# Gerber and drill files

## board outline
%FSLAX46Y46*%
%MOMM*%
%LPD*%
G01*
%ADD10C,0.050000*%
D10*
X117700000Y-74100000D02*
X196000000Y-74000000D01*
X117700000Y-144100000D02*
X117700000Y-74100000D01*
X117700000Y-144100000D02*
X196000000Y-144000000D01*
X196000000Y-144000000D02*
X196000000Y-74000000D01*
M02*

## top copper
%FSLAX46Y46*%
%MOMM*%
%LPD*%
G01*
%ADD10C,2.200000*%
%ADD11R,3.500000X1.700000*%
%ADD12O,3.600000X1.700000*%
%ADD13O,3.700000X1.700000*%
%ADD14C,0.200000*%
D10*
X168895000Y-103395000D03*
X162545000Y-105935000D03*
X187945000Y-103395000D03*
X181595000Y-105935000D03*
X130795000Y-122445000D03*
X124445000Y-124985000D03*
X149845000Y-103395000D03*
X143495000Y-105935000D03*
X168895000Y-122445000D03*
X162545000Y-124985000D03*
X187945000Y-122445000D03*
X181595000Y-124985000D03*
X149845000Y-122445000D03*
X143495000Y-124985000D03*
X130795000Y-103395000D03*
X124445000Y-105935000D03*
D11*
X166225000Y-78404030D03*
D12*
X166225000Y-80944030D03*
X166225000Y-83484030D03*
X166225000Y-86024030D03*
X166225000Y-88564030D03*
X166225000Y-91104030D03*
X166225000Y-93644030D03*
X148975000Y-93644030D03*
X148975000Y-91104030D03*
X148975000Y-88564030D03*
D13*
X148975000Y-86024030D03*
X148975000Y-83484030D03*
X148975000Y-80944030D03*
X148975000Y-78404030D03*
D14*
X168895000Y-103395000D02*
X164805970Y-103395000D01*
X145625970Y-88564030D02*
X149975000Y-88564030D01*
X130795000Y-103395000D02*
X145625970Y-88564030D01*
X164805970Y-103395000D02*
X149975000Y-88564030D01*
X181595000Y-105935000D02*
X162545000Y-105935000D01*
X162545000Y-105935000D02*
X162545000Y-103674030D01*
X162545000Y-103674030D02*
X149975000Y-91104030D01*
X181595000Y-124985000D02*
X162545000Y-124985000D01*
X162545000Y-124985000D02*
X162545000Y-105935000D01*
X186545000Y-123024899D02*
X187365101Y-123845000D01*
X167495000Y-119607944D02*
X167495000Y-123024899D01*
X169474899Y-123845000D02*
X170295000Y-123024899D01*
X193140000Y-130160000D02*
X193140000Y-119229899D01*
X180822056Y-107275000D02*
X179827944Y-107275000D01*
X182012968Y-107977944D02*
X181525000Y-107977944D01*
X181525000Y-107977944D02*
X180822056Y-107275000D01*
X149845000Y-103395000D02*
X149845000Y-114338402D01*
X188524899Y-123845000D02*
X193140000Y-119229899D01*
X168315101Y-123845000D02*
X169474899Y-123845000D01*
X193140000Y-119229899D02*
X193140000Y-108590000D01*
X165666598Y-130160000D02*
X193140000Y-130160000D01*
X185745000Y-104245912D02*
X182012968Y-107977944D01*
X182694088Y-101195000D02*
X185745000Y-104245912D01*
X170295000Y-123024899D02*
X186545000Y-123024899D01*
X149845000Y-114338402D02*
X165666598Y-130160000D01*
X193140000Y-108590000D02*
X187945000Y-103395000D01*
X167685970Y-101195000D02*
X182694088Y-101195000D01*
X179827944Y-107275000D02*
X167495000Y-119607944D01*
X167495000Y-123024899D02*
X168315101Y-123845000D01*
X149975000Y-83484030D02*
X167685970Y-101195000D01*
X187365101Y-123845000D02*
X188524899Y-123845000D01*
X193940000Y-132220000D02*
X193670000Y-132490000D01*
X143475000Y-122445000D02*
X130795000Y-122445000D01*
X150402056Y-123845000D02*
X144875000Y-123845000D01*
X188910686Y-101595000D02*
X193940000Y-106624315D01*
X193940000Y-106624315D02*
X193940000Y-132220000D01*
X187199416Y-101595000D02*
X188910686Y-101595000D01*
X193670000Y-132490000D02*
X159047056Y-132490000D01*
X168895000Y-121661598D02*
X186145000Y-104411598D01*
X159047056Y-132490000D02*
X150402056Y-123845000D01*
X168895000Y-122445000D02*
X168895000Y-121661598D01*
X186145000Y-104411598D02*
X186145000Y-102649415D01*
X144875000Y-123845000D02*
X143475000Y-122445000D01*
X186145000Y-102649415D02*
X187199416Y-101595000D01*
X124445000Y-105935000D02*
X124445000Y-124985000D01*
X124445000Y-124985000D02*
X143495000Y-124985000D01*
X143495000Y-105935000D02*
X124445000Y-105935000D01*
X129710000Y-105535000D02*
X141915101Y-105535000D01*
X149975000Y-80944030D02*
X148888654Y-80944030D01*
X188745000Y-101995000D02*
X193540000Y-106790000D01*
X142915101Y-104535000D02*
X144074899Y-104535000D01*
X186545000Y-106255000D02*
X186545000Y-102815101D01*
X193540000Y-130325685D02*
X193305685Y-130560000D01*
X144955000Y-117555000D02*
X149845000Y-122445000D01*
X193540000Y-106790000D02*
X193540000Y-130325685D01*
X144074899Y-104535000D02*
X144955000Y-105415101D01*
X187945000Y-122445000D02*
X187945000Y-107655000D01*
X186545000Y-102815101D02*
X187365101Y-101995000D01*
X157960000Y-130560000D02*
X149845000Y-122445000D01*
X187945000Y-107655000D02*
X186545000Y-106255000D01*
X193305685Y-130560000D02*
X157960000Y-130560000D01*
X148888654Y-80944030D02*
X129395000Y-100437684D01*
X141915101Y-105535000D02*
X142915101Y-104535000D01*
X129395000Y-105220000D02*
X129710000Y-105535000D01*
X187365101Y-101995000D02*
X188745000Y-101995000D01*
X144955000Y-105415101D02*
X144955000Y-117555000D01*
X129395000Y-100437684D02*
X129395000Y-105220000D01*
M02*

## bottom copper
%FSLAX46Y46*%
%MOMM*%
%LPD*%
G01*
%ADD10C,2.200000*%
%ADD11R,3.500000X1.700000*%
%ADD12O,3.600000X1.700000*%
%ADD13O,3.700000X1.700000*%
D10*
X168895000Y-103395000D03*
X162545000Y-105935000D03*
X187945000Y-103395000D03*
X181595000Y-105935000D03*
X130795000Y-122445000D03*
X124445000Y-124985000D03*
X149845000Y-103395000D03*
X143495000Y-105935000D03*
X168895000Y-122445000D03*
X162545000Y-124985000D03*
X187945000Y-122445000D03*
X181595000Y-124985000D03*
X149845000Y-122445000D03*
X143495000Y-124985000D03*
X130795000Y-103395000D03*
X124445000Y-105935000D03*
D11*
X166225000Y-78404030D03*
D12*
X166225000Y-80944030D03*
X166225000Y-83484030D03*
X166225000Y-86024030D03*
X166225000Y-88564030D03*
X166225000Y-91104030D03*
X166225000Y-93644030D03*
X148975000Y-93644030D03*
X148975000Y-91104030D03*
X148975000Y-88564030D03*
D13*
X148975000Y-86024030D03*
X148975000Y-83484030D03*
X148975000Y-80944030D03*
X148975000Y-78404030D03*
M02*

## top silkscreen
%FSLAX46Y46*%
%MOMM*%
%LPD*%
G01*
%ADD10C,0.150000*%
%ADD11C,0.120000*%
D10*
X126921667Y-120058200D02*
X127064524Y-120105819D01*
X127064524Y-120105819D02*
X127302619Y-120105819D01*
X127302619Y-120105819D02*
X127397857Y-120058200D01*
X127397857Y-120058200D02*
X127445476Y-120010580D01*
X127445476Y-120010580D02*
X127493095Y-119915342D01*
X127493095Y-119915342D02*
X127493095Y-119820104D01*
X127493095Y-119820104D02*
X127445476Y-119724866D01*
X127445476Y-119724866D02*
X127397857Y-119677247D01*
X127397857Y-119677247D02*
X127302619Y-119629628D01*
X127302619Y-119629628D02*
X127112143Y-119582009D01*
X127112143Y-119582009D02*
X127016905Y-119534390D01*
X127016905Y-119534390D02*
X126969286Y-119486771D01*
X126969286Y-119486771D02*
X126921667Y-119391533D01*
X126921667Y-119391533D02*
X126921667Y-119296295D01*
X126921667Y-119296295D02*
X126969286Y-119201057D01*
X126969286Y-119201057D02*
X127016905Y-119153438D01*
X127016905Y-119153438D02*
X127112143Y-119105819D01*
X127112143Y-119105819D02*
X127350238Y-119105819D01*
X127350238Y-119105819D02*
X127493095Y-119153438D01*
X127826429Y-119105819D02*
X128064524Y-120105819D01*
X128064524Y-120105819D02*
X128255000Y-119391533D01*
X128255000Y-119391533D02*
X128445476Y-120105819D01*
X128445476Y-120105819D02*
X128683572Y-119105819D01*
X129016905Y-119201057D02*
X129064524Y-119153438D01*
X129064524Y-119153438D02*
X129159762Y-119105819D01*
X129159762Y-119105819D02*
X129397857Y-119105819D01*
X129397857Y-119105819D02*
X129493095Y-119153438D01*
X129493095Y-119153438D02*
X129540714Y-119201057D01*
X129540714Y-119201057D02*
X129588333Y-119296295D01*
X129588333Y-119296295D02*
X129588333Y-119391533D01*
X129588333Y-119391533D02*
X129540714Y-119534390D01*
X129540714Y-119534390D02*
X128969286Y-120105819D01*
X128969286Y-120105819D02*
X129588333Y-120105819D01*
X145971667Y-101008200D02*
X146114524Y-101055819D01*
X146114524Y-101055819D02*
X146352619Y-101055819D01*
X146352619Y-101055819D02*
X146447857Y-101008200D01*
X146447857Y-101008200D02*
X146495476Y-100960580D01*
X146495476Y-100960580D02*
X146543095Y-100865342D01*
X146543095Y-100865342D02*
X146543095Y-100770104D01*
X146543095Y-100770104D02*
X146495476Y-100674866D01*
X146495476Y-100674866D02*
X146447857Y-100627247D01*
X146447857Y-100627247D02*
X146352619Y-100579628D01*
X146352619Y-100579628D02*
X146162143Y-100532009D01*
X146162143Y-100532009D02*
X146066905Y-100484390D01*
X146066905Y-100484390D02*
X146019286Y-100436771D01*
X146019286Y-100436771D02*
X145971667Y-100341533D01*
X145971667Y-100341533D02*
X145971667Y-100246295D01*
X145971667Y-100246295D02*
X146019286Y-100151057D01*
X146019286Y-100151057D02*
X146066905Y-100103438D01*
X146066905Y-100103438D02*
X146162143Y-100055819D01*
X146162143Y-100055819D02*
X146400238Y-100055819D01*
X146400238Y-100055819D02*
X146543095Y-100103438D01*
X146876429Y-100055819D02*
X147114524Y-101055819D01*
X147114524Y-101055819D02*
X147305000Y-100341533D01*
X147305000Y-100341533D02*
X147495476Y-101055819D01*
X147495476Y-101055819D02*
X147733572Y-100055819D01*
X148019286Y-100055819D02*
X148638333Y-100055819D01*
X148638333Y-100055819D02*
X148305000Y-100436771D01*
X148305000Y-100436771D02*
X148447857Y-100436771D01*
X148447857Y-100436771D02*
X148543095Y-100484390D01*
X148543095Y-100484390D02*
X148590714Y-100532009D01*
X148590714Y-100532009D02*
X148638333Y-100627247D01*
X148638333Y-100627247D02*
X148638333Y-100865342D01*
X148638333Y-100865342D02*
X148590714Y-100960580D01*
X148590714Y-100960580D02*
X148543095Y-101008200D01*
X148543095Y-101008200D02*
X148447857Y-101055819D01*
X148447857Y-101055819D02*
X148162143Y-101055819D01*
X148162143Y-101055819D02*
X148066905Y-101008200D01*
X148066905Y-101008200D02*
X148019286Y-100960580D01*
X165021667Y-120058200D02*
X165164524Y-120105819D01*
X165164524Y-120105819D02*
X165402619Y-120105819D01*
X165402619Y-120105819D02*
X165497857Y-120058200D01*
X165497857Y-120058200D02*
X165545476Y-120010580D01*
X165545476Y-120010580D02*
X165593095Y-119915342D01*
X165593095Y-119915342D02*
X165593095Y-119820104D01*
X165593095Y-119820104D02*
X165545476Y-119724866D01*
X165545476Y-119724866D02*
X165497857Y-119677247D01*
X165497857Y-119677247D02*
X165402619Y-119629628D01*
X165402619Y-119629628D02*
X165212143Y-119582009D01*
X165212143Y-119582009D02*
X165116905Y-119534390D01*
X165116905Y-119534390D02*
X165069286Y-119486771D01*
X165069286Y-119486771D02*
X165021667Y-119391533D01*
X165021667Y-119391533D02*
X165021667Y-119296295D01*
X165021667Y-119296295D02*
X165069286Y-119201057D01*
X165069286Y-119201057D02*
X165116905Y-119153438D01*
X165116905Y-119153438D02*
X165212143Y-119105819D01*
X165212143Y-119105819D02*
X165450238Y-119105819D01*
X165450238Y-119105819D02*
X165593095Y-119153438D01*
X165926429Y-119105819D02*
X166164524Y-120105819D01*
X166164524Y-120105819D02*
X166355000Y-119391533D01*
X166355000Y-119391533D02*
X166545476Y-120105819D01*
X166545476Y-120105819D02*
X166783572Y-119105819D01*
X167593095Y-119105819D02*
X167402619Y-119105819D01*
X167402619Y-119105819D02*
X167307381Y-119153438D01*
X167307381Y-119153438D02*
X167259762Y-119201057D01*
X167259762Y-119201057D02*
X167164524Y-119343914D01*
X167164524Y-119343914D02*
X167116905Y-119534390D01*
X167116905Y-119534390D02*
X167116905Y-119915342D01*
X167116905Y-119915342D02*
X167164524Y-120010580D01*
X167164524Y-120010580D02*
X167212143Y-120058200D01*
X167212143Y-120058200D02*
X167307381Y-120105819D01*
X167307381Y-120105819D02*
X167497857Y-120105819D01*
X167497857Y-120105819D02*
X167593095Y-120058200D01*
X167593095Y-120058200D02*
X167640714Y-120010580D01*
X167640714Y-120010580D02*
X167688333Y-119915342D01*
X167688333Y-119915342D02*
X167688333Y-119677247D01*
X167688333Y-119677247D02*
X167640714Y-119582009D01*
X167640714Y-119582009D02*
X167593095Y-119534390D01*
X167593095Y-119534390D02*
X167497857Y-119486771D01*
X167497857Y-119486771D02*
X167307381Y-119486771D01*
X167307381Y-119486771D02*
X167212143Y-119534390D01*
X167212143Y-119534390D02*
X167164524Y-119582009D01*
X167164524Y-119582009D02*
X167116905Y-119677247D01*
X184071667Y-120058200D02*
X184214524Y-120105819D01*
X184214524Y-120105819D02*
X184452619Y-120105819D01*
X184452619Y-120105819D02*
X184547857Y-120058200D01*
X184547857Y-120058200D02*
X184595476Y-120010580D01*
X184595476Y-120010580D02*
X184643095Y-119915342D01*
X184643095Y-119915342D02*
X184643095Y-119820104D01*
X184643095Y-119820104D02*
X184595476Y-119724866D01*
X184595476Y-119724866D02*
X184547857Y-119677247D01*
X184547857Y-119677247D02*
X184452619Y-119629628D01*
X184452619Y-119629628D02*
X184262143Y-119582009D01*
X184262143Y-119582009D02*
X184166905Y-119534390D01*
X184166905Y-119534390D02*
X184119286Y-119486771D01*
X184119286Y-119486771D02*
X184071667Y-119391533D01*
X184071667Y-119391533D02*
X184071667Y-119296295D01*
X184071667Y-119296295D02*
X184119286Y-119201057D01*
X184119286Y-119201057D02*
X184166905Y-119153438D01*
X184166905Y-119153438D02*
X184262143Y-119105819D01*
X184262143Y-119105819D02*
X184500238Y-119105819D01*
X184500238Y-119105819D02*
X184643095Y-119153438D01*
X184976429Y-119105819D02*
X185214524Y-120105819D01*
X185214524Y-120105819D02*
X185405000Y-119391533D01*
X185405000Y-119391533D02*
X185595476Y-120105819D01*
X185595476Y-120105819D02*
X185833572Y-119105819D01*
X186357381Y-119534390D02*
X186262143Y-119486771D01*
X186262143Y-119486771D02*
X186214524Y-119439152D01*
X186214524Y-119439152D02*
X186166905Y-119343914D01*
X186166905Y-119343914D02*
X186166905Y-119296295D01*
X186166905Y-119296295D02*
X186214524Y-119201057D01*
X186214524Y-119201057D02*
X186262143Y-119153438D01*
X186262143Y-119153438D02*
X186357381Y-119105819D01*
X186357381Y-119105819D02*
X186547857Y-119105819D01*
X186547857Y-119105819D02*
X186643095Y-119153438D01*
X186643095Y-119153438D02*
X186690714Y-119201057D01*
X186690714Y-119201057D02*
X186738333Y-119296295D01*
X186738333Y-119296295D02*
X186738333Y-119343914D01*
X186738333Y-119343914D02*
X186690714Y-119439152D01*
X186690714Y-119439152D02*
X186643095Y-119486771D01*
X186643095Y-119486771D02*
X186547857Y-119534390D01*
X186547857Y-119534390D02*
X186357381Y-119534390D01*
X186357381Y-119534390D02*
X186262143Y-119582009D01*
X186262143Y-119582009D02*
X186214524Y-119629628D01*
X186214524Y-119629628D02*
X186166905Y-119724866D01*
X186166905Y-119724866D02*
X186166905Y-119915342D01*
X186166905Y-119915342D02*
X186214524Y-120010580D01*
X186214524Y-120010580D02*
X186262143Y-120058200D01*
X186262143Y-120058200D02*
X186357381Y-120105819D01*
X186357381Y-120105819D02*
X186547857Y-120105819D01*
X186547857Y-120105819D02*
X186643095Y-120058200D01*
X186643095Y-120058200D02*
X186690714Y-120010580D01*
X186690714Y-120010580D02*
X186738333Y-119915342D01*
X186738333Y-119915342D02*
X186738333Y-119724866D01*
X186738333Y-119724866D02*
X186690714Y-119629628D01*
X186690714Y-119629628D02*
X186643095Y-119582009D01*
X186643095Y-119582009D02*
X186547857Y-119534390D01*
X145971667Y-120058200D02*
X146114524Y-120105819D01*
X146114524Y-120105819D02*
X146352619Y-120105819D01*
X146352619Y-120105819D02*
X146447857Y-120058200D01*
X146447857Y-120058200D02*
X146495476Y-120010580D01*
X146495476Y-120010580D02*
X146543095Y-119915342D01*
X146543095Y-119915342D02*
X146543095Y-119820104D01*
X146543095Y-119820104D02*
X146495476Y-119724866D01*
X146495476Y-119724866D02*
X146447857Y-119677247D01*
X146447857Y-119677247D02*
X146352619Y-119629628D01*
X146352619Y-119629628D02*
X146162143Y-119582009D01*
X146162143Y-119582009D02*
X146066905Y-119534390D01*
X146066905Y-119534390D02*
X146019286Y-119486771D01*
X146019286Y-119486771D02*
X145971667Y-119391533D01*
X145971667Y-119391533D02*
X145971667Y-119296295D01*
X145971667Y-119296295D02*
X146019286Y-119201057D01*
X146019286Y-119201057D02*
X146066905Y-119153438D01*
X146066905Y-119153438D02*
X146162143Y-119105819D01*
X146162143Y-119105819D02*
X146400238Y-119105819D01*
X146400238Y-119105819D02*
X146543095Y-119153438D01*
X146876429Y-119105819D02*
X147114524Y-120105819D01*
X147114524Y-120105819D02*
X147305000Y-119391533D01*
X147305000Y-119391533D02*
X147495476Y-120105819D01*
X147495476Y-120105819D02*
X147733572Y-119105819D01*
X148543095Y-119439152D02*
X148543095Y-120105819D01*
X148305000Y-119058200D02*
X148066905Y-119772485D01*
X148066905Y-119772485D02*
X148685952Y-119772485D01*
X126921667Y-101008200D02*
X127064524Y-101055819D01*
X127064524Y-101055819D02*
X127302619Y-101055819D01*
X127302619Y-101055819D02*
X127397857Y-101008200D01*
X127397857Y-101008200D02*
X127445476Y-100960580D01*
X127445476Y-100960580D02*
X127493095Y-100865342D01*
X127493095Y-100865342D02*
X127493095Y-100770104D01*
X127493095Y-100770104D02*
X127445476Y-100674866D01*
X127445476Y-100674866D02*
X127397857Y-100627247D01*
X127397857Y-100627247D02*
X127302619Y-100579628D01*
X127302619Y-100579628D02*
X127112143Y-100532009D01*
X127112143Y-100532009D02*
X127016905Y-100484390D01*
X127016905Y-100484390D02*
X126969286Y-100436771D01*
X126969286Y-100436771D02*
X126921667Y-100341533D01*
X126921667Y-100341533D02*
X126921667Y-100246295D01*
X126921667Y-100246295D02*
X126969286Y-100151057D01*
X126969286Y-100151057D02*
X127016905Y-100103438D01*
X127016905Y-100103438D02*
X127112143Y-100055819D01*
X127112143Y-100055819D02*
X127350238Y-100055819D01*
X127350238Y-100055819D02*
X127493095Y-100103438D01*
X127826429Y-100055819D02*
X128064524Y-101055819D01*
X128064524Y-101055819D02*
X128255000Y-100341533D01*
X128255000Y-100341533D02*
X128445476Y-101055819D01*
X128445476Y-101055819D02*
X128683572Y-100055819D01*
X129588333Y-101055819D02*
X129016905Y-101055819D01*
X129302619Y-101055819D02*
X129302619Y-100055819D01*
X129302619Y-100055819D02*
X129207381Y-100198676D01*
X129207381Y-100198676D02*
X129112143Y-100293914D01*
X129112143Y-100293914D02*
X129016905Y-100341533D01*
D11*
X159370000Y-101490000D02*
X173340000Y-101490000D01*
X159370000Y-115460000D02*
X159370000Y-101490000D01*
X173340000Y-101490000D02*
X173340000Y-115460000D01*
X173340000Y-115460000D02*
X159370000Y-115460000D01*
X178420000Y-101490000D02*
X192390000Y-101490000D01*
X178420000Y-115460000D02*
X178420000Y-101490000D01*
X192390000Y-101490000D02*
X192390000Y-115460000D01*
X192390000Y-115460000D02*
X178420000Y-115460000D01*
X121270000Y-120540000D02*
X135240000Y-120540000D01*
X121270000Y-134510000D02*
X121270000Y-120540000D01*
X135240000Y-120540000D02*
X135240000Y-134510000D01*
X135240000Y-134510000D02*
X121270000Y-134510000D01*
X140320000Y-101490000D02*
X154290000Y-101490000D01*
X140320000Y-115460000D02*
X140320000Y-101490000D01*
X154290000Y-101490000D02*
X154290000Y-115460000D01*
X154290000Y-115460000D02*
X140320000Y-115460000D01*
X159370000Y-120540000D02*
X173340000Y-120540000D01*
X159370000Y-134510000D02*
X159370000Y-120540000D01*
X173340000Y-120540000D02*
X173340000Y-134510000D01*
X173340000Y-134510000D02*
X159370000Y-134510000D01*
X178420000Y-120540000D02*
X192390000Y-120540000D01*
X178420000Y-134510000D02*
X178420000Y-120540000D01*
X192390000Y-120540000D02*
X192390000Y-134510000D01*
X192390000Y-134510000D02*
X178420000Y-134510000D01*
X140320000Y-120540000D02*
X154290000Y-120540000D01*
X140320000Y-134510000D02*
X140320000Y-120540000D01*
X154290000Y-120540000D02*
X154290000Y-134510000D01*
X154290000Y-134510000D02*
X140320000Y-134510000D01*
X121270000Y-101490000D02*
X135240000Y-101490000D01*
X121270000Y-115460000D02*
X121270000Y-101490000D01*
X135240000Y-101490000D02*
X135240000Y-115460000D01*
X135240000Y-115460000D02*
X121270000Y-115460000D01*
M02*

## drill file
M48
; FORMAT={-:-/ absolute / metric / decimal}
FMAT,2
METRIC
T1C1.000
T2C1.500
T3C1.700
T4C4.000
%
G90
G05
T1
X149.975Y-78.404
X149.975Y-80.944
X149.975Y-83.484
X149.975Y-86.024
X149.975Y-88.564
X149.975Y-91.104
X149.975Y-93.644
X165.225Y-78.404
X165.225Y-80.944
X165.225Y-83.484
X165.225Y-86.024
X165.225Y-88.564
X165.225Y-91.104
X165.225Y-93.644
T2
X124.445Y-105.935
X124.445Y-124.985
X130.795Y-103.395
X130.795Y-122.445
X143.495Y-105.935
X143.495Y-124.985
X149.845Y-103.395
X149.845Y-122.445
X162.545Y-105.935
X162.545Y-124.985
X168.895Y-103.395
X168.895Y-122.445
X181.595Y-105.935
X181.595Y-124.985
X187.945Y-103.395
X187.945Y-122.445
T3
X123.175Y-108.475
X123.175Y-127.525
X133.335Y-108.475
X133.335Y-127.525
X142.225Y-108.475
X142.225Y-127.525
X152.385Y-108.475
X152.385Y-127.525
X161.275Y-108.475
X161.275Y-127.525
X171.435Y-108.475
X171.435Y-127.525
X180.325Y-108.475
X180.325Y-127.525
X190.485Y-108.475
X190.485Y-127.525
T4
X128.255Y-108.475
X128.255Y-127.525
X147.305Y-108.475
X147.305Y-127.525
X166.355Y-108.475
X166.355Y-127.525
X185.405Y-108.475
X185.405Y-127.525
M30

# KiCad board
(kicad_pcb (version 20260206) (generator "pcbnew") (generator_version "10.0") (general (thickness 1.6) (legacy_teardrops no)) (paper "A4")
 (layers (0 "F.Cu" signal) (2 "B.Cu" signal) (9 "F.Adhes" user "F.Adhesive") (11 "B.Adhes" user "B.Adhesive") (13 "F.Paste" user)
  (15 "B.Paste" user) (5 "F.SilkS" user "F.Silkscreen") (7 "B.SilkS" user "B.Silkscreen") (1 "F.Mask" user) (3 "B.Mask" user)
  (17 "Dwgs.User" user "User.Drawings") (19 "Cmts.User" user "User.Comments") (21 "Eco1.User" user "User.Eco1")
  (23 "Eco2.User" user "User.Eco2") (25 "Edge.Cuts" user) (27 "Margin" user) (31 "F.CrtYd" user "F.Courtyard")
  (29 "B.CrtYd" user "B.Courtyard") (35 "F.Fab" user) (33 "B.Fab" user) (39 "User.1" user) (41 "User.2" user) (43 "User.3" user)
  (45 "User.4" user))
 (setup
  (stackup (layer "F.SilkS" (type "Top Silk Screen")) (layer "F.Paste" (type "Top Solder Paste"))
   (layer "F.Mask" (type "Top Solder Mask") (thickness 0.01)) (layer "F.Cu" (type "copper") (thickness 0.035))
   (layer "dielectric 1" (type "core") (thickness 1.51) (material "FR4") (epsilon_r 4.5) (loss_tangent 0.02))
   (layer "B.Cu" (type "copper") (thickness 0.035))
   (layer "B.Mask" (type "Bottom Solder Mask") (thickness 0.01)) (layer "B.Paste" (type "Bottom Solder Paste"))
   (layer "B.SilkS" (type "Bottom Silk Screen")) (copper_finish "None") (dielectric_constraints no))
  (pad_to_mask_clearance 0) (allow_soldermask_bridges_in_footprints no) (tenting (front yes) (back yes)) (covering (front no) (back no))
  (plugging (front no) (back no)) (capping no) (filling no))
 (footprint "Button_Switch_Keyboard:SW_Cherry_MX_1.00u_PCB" (layer "F.Cu") (at 168.895 103.395)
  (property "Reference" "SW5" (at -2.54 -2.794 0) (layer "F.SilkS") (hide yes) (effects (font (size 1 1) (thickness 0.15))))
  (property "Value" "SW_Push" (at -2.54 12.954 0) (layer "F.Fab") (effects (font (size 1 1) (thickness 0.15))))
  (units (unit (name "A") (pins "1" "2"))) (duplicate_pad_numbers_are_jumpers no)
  (fp_line (start -9.525 -1.905) (end 4.445 -1.905) (stroke (width 0.12) (type solid)) (layer "F.SilkS"))
  (fp_line (start -9.525 12.065) (end -9.525 -1.905) (stroke (width 0.12) (type solid)) (layer "F.SilkS"))
  (fp_line (start 4.445 -1.905) (end 4.445 12.065) (stroke (width 0.12) (type solid)) (layer "F.SilkS"))
  (fp_line (start 4.445 12.065) (end -9.525 12.065) (stroke (width 0.12) (type solid)) (layer "F.SilkS"))
  (pad "" np_thru_hole circle (at -7.62 5.08) (size 1.7 1.7) (drill 1.7) (layers "*.Cu" "*.Mask"))
  (pad "" np_thru_hole circle (at -2.54 5.08) (size 4 4) (drill 4) (layers "*.Cu" "*.Mask"))
  (pad "" np_thru_hole circle (at 2.54 5.08) (size 1.7 1.7) (drill 1.7) (layers "*.Cu" "*.Mask"))
  (pad "1" thru_hole circle (at 0 0) (size 2.2 2.2) (drill 1.5) (layers "*.Cu" "*.Mask") (remove_unused_layers no)
   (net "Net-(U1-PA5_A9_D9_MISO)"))
  (pad "2" thru_hole circle (at -6.35 2.54) (size 2.2 2.2) (drill 1.5) (layers "*.Cu" "*.Mask") (remove_unused_layers no)
   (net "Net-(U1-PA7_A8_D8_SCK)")))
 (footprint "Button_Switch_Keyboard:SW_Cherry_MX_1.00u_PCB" (layer "F.Cu") (at 187.945 103.395)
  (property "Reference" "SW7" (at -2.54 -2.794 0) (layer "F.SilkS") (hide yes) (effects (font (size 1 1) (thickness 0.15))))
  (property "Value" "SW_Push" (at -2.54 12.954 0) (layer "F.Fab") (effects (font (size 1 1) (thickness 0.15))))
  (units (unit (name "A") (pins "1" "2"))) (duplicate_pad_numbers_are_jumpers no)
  (fp_line (start -9.525 -1.905) (end 4.445 -1.905) (stroke (width 0.12) (type solid)) (layer "F.SilkS"))
  (fp_line (start -9.525 12.065) (end -9.525 -1.905) (stroke (width 0.12) (type solid)) (layer "F.SilkS"))
  (fp_line (start 4.445 -1.905) (end 4.445 12.065) (stroke (width 0.12) (type solid)) (layer "F.SilkS"))
  (fp_line (start 4.445 12.065) (end -9.525 12.065) (stroke (width 0.12) (type solid)) (layer "F.SilkS"))
  (pad "" np_thru_hole circle (at -7.62 5.08) (size 1.7 1.7) (drill 1.7) (layers "*.Cu" "*.Mask"))
  (pad "" np_thru_hole circle (at -2.54 5.08) (size 4 4) (drill 4) (layers "*.Cu" "*.Mask"))
  (pad "" np_thru_hole circle (at 2.54 5.08) (size 1.7 1.7) (drill 1.7) (layers "*.Cu" "*.Mask"))
  (pad "1" thru_hole circle (at 0 0) (size 2.2 2.2) (drill 1.5) (layers "*.Cu" "*.Mask") (remove_unused_layers no) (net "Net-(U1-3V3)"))
  (pad "2" thru_hole circle (at -6.35 2.54) (size 2.2 2.2) (drill 1.5) (layers "*.Cu" "*.Mask") (remove_unused_layers no)
   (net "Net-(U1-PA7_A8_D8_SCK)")))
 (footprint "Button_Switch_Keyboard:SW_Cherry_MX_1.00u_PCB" (layer "F.Cu") (at 130.795 122.445)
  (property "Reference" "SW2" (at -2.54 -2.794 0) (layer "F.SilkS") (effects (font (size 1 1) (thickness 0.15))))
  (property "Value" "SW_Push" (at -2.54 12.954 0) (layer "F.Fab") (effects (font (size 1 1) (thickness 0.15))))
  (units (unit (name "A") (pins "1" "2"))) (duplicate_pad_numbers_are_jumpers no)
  (fp_line (start -9.525 -1.905) (end 4.445 -1.905) (stroke (width 0.12) (type solid)) (layer "F.SilkS"))
  (fp_line (start -9.525 12.065) (end -9.525 -1.905) (stroke (width 0.12) (type solid)) (layer "F.SilkS"))
  (fp_line (start 4.445 -1.905) (end 4.445 12.065) (stroke (width 0.12) (type solid)) (layer "F.SilkS"))
  (fp_line (start 4.445 12.065) (end -9.525 12.065) (stroke (width 0.12) (type solid)) (layer "F.SilkS"))
  (pad "" np_thru_hole circle (at -7.62 5.08) (size 1.7 1.7) (drill 1.7) (layers "*.Cu" "*.Mask"))
  (pad "" np_thru_hole circle (at -2.54 5.08) (size 4 4) (drill 4) (layers "*.Cu" "*.Mask"))
  (pad "" np_thru_hole circle (at 2.54 5.08) (size 1.7 1.7) (drill 1.7) (layers "*.Cu" "*.Mask"))
  (pad "1" thru_hole circle (at 0 0) (size 2.2 2.2) (drill 1.5) (layers "*.Cu" "*.Mask") (remove_unused_layers no)
   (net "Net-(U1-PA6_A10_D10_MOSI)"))
  (pad "2" thru_hole circle (at -6.35 2.54) (size 2.2 2.2) (drill 1.5) (layers "*.Cu" "*.Mask") (remove_unused_layers no)
   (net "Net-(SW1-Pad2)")))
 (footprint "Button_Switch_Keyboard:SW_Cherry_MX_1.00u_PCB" (layer "F.Cu") (at 149.845 103.395)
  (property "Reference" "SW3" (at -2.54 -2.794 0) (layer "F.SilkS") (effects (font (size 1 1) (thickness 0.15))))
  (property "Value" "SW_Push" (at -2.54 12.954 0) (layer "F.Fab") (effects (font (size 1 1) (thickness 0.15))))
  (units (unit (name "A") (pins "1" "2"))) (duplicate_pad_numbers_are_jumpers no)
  (fp_line (start -9.525 -1.905) (end 4.445 -1.905) (stroke (width 0.12) (type solid)) (layer "F.SilkS"))
  (fp_line (start -9.525 12.065) (end -9.525 -1.905) (stroke (width 0.12) (type solid)) (layer "F.SilkS"))
  (fp_line (start 4.445 -1.905) (end 4.445 12.065) (stroke (width 0.12) (type solid)) (layer "F.SilkS"))
  (fp_line (start 4.445 12.065) (end -9.525 12.065) (stroke (width 0.12) (type solid)) (layer "F.SilkS"))
  (pad "" np_thru_hole circle (at -7.62 5.08) (size 1.7 1.7) (drill 1.7) (layers "*.Cu" "*.Mask"))
  (pad "" np_thru_hole circle (at -2.54 5.08) (size 4 4) (drill 4) (layers "*.Cu" "*.Mask"))
  (pad "" np_thru_hole circle (at 2.54 5.08) (size 1.7 1.7) (drill 1.7) (layers "*.Cu" "*.Mask"))
  (pad "1" thru_hole circle (at 0 0) (size 2.2 2.2) (drill 1.5) (layers "*.Cu" "*.Mask") (remove_unused_layers no) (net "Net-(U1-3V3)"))
  (pad "2" thru_hole circle (at -6.35 2.54) (size 2.2 2.2) (drill 1.5) (layers "*.Cu" "*.Mask") (remove_unused_layers no)
   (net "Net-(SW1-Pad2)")))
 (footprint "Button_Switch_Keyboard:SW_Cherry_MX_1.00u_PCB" (layer "F.Cu") (at 168.895 122.445)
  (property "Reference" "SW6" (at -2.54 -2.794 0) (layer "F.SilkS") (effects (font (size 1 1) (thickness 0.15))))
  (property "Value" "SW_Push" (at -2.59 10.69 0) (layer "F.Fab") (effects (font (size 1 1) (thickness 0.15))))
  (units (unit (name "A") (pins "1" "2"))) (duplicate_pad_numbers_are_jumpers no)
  (fp_line (start -9.525 -1.905) (end 4.445 -1.905) (stroke (width 0.12) (type solid)) (layer "F.SilkS"))
  (fp_line (start -9.525 12.065) (end -9.525 -1.905) (stroke (width 0.12) (type solid)) (layer "F.SilkS"))
  (fp_line (start 4.445 -1.905) (end 4.445 12.065) (stroke (width 0.12) (type solid)) (layer "F.SilkS"))
  (fp_line (start 4.445 12.065) (end -9.525 12.065) (stroke (width 0.12) (type solid)) (layer "F.SilkS"))
  (pad "" np_thru_hole circle (at -7.62 5.08) (size 1.7 1.7) (drill 1.7) (layers "*.Cu" "*.Mask"))
  (pad "" np_thru_hole circle (at -2.54 5.08) (size 4 4) (drill 4) (layers "*.Cu" "*.Mask"))
  (pad "" np_thru_hole circle (at 2.54 5.08) (size 1.7 1.7) (drill 1.7) (layers "*.Cu" "*.Mask"))
  (pad "1" thru_hole circle (at 0 0) (size 2.2 2.2) (drill 1.5) (layers "*.Cu" "*.Mask") (remove_unused_layers no)
   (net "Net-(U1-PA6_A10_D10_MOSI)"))
  (pad "2" thru_hole circle (at -6.35 2.54) (size 2.2 2.2) (drill 1.5) (layers "*.Cu" "*.Mask") (remove_unused_layers no)
   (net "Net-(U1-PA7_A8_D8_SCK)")))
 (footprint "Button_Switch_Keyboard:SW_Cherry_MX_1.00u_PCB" (layer "F.Cu") (at 187.945 122.445)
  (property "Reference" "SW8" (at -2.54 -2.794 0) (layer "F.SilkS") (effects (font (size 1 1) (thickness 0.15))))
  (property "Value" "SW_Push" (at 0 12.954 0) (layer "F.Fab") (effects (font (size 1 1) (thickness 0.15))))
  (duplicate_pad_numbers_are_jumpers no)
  (fp_line (start -9.525 -1.905) (end 4.445 -1.905) (stroke (width 0.12) (type solid)) (layer "F.SilkS"))
  (fp_line (start -9.525 12.065) (end -9.525 -1.905) (stroke (width 0.12) (type solid)) (layer "F.SilkS"))
  (fp_line (start 4.445 -1.905) (end 4.445 12.065) (stroke (width 0.12) (type solid)) (layer "F.SilkS"))
  (fp_line (start 4.445 12.065) (end -9.525 12.065) (stroke (width 0.12) (type solid)) (layer "F.SilkS"))
  (pad "" np_thru_hole circle (at -7.62 5.08) (size 1.7 1.7) (drill 1.7) (layers "*.Cu" "*.Mask"))
  (pad "" np_thru_hole circle (at -2.54 5.08) (size 4 4) (drill 4) (layers "*.Cu" "*.Mask"))
  (pad "" np_thru_hole circle (at 2.54 5.08) (size 1.7 1.7) (drill 1.7) (layers "*.Cu" "*.Mask"))
  (pad "1" thru_hole circle (at 0 0) (size 2.2 2.2) (drill 1.5) (layers "*.Cu" "*.Mask") (remove_unused_layers no) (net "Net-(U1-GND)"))
  (pad "2" thru_hole circle (at -6.35 2.54) (size 2.2 2.2) (drill 1.5) (layers "*.Cu" "*.Mask") (remove_unused_layers no)
   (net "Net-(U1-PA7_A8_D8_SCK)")))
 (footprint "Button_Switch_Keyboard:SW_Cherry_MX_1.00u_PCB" (layer "F.Cu") (at 149.845 122.445)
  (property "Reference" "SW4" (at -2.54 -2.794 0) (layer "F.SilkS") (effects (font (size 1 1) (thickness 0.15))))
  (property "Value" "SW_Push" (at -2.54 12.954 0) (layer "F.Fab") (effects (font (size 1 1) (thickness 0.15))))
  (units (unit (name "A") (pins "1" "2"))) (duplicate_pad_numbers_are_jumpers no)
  (fp_line (start -9.525 -1.905) (end 4.445 -1.905) (stroke (width 0.12) (type solid)) (layer "F.SilkS"))
  (fp_line (start -9.525 12.065) (end -9.525 -1.905) (stroke (width 0.12) (type solid)) (layer "F.SilkS"))
  (fp_line (start 4.445 -1.905) (end 4.445 12.065) (stroke (width 0.12) (type solid)) (layer "F.SilkS"))
  (fp_line (start 4.445 12.065) (end -9.525 12.065) (stroke (width 0.12) (type solid)) (layer "F.SilkS"))
  (pad "" np_thru_hole circle (at -7.62 5.08) (size 1.7 1.7) (drill 1.7) (layers "*.Cu" "*.Mask"))
  (pad "" np_thru_hole circle (at -2.54 5.08) (size 4 4) (drill 4) (layers "*.Cu" "*.Mask"))
  (pad "" np_thru_hole circle (at 2.54 5.08) (size 1.7 1.7) (drill 1.7) (layers "*.Cu" "*.Mask"))
  (pad "1" thru_hole circle (at 0 0) (size 2.2 2.2) (drill 1.5) (layers "*.Cu" "*.Mask") (remove_unused_layers no) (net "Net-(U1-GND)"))
  (pad "2" thru_hole circle (at -6.35 2.54) (size 2.2 2.2) (drill 1.5) (layers "*.Cu" "*.Mask") (remove_unused_layers no)
   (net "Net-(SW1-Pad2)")))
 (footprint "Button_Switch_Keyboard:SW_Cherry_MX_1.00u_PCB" (layer "F.Cu") (at 130.795 103.395)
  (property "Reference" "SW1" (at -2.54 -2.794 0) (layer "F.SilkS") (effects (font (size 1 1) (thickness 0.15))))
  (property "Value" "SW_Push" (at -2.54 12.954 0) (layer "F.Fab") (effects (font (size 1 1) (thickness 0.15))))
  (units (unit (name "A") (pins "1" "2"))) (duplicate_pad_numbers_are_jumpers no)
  (fp_line (start -9.525 -1.905) (end 4.445 -1.905) (stroke (width 0.12) (type solid)) (layer "F.SilkS"))
  (fp_line (start -9.525 12.065) (end -9.525 -1.905) (stroke (width 0.12) (type solid)) (layer "F.SilkS"))
  (fp_line (start 4.445 -1.905) (end 4.445 12.065) (stroke (width 0.12) (type solid)) (layer "F.SilkS"))
  (fp_line (start 4.445 12.065) (end -9.525 12.065) (stroke (width 0.12) (type solid)) (layer "F.SilkS"))
  (pad "" np_thru_hole circle (at -7.62 5.08) (size 1.7 1.7) (drill 1.7) (layers "*.Cu" "*.Mask"))
  (pad "" np_thru_hole circle (at -2.54 5.08) (size 4 4) (drill 4) (layers "*.Cu" "*.Mask"))
  (pad "" np_thru_hole circle (at 2.54 5.08) (size 1.7 1.7) (drill 1.7) (layers "*.Cu" "*.Mask"))
  (pad "1" thru_hole circle (at 0 0) (size 2.2 2.2) (drill 1.5) (layers "*.Cu" "*.Mask") (remove_unused_layers no)
   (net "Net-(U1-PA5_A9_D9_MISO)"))
  (pad "2" thru_hole circle (at -6.35 2.54) (size 2.2 2.2) (drill 1.5) (layers "*.Cu" "*.Mask") (remove_unused_layers no)
   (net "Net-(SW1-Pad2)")))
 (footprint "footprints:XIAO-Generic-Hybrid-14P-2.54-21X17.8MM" (layer "B.Cu") (at 157.6 86.02403 180)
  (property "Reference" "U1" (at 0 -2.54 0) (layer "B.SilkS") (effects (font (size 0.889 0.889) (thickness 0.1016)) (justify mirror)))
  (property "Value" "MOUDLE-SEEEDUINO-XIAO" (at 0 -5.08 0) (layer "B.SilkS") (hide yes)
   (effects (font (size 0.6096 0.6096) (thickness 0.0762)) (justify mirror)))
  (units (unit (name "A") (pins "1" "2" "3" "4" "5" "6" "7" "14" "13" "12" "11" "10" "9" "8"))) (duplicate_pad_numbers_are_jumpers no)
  (pad "1" thru_hole rect (at -7.625 7.62 180) (size 3.5 1.7) (drill 1 (offset -1 0)) (layers "*.Cu" "*.Mask") (remove_unused_layers no)
   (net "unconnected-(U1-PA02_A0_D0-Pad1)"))
  (pad "2" thru_hole oval (at -7.625 5.08 180) (size 3.6 1.7) (drill 1 (offset -1 0)) (layers "*.Cu" "*.Mask") (remove_unused_layers no)
   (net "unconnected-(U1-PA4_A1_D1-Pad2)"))
  (pad "3" thru_hole oval (at -7.625 2.54 180) (size 3.6 1.7) (drill 1 (offset -1 0)) (layers "*.Cu" "*.Mask") (remove_unused_layers no)
   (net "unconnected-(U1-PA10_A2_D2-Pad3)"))
  (pad "4" thru_hole oval (at -7.625 0 180) (size 3.6 1.7) (drill 1 (offset -1 0)) (layers "*.Cu" "*.Mask") (remove_unused_layers no)
   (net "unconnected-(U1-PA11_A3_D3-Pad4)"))
  (pad "5" thru_hole oval (at -7.625 -2.54 180) (size 3.6 1.7) (drill 1 (offset -1 0)) (layers "*.Cu" "*.Mask") (remove_unused_layers no)
   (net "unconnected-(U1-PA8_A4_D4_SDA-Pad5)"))
  (pad "6" thru_hole oval (at -7.625 -5.08) (size 3.6 1.7) (drill 1 (offset 1 0)) (layers "*.Cu" "*.Mask") (remove_unused_layers no)
   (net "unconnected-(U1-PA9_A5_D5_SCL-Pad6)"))
  (pad "7" thru_hole oval (at -7.625 -7.62 180) (size 3.6 1.7) (drill 1 (offset -1 0)) (layers "*.Cu" "*.Mask") (remove_unused_layers no)
   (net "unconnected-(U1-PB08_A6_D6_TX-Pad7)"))
  (pad "8" thru_hole oval (at 7.625 -7.62 180) (size 3.6 1.7) (drill 1 (offset 1 0)) (layers "*.Cu" "*.Mask") (remove_unused_layers no)
   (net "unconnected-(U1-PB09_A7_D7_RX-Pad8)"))
  (pad "9" thru_hole oval (at 7.625 -5.08 180) (size 3.6 1.7) (drill 1 (offset 1 0)) (layers "*.Cu" "*.Mask") (remove_unused_layers no)
   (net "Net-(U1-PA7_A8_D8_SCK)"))
  (pad "10" thru_hole oval (at 7.625 -2.54 180) (size 3.6 1.7) (drill 1 (offset 1 0)) (layers "*.Cu" "*.Mask") (remove_unused_layers no)
   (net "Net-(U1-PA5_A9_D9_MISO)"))
  (pad "11" thru_hole oval (at 7.625 0 180) (size 3.7 1.7) (drill 1 (offset 1 0)) (layers "*.Cu" "*.Mask") (remove_unused_layers no)
   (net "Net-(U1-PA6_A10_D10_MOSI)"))
  (pad "12" thru_hole oval (at 7.625 2.54 180) (size 3.7 1.7) (drill 1 (offset 1 0)) (layers "*.Cu" "*.Mask") (remove_unused_layers no)
   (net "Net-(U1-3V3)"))
  (pad "13" thru_hole oval (at 7.625 5.08 180) (size 3.7 1.7) (drill 1 (offset 1 0)) (layers "*.Cu" "*.Mask") (remove_unused_layers no)
   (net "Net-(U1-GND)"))
  (pad "14" thru_hole oval (at 7.625 7.62 180) (size 3.7 1.7) (drill 1 (offset 1 0)) (layers "*.Cu" "*.Mask") (remove_unused_layers no)
   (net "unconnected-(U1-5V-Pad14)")))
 (gr_line (start 117.7 74.1) (end 196 74) (stroke (width 0.05) (type default)) (layer "Edge.Cuts"))
 (gr_line (start 117.7 144.1) (end 117.7 74.1) (stroke (width 0.05) (type default)) (layer "Edge.Cuts"))
 (gr_line (start 117.7 144.1) (end 196 144) (stroke (width 0.05) (type default)) (layer "Edge.Cuts"))
 (gr_line (start 196 144) (end 196 74) (stroke (width 0.05) (type default)) (layer "Edge.Cuts"))
 (segment (start 168.895 103.395) (end 164.80597 103.395) (width 0.2) (layer "F.Cu") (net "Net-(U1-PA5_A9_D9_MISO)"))
 (segment (start 145.62597 88.56403) (end 149.975 88.56403) (width 0.2) (layer "F.Cu") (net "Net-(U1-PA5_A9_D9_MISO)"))
 (segment (start 130.795 103.395) (end 145.62597 88.56403) (width 0.2) (layer "F.Cu") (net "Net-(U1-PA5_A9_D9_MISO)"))
 (segment (start 164.80597 103.395) (end 149.975 88.56403) (width 0.2) (layer "F.Cu") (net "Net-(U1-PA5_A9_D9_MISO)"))
 (segment (start 181.595 105.935) (end 162.545 105.935) (width 0.2) (layer "F.Cu") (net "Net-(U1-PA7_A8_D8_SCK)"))
 (segment (start 162.545 105.935) (end 162.545 103.67403) (width 0.2) (layer "F.Cu") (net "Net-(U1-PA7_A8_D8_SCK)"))
 (segment (start 162.545 103.67403) (end 149.975 91.10403) (width 0.2) (layer "F.Cu") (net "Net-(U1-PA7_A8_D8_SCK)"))
 (segment (start 181.595 124.985) (end 162.545 124.985) (width 0.2) (layer "F.Cu") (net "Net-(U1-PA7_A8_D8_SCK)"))
 (segment (start 162.545 124.985) (end 162.545 105.935) (width 0.2) (layer "F.Cu") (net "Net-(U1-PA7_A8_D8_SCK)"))
 (segment (start 186.545 123.024899) (end 187.365101 123.845) (width 0.2) (layer "F.Cu") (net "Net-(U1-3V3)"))
 (segment (start 167.495 119.607944) (end 167.495 123.024899) (width 0.2) (layer "F.Cu") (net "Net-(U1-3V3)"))
 (segment (start 169.474899 123.845) (end 170.295 123.024899) (width 0.2) (layer "F.Cu") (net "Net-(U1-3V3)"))
 (segment (start 193.14 130.16) (end 193.14 119.229899) (width 0.2) (layer "F.Cu") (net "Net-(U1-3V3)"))
 (segment (start 180.822056 107.275) (end 179.827944 107.275) (width 0.2) (layer "F.Cu") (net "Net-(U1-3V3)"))
 (segment (start 182.012968 107.977944) (end 181.525 107.977944) (width 0.2) (layer "F.Cu") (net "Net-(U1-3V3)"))
 (segment (start 181.525 107.977944) (end 180.822056 107.275) (width 0.2) (layer "F.Cu") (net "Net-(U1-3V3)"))
 (segment (start 149.845 103.395) (end 149.845 114.338402) (width 0.2) (layer "F.Cu") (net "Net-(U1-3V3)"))
 (segment (start 188.524899 123.845) (end 193.14 119.229899) (width 0.2) (layer "F.Cu") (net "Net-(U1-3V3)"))
 (segment (start 168.315101 123.845) (end 169.474899 123.845) (width 0.2) (layer "F.Cu") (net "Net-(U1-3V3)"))
 (segment (start 193.14 119.229899) (end 193.14 108.59) (width 0.2) (layer "F.Cu") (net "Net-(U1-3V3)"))
 (segment (start 165.666598 130.16) (end 193.14 130.16) (width 0.2) (layer "F.Cu") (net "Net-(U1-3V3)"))
 (segment (start 185.745 104.245912) (end 182.012968 107.977944) (width 0.2) (layer "F.Cu") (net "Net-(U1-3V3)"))
 (segment (start 182.694088 101.195) (end 185.745 104.245912) (width 0.2) (layer "F.Cu") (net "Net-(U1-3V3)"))
 (segment (start 170.295 123.024899) (end 186.545 123.024899) (width 0.2) (layer "F.Cu") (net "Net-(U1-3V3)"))
 (segment (start 149.845 114.338402) (end 165.666598 130.16) (width 0.2) (layer "F.Cu") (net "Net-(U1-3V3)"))
 (segment (start 193.14 108.59) (end 187.945 103.395) (width 0.2) (layer "F.Cu") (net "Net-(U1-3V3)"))
 (segment (start 167.68597 101.195) (end 182.694088 101.195) (width 0.2) (layer "F.Cu") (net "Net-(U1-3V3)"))
 (segment (start 179.827944 107.275) (end 167.495 119.607944) (width 0.2) (layer "F.Cu") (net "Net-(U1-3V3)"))
 (segment (start 167.495 123.024899) (end 168.315101 123.845) (width 0.2) (layer "F.Cu") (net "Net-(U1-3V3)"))
 (segment (start 149.975 83.48403) (end 167.68597 101.195) (width 0.2) (layer "F.Cu") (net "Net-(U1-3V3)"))
 (segment (start 187.365101 123.845) (end 188.524899 123.845) (width 0.2) (layer "F.Cu") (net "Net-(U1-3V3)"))
 (segment (start 193.94 132.22) (end 193.67 132.49) (width 0.2) (layer "F.Cu") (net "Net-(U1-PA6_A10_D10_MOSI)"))
 (segment (start 143.475 122.445) (end 130.795 122.445) (width 0.2) (layer "F.Cu") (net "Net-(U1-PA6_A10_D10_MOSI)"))
 (segment (start 150.402056 123.845) (end 144.875 123.845) (width 0.2) (layer "F.Cu") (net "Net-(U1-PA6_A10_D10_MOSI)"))
 (segment (start 188.910686 101.595) (end 193.94 106.624315) (width 0.2) (layer "F.Cu") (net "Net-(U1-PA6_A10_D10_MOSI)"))
 (segment (start 193.94 106.624315) (end 193.94 132.22) (width 0.2) (layer "F.Cu") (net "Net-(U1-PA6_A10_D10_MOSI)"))
 (segment (start 187.199416 101.595) (end 188.910686 101.595) (width 0.2) (layer "F.Cu") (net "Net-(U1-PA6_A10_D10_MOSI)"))
 (segment (start 193.67 132.49) (end 159.047056 132.49) (width 0.2) (layer "F.Cu") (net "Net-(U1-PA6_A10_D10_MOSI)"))
 (segment (start 168.895 121.661598) (end 186.145 104.411598) (width 0.2) (layer "F.Cu") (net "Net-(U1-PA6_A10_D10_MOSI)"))
 (segment (start 159.047056 132.49) (end 150.402056 123.845) (width 0.2) (layer "F.Cu") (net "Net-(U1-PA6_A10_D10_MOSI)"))
 (segment (start 168.895 122.445) (end 168.895 121.661598) (width 0.2) (layer "F.Cu") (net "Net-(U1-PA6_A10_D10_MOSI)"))
 (segment (start 186.145 104.411598) (end 186.145 102.649415) (width 0.2) (layer "F.Cu") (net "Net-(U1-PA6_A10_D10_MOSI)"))
 (segment (start 144.875 123.845) (end 143.475 122.445) (width 0.2) (layer "F.Cu") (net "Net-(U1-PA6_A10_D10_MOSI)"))
 (segment (start 186.145 102.649415) (end 187.199416 101.595) (width 0.2) (layer "F.Cu") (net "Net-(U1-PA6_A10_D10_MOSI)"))
 (segment (start 124.445 105.935) (end 124.445 124.985) (width 0.2) (layer "F.Cu") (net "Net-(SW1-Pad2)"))
 (segment (start 124.445 124.985) (end 143.495 124.985) (width 0.2) (layer "F.Cu") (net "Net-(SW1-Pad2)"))
 (segment (start 143.495 105.935) (end 124.445 105.935) (width 0.2) (layer "F.Cu") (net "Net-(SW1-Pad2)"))
 (segment (start 129.71 105.535) (end 141.915101 105.535) (width 0.2) (layer "F.Cu") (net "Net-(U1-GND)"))
 (segment (start 149.975 80.94403) (end 148.888654 80.94403) (width 0.2) (layer "F.Cu") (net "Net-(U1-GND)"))
 (segment (start 188.745 101.995) (end 193.54 106.79) (width 0.2) (layer "F.Cu") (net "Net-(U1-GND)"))
 (segment (start 142.915101 104.535) (end 144.074899 104.535) (width 0.2) (layer "F.Cu") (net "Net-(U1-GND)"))
 (segment (start 186.545 106.255) (end 186.545 102.815101) (width 0.2) (layer "F.Cu") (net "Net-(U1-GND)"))
 (segment (start 193.54 130.325685) (end 193.305685 130.56) (width 0.2) (layer "F.Cu") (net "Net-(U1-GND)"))
 (segment (start 144.955 117.555) (end 149.845 122.445) (width 0.2) (layer "F.Cu") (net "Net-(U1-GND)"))
 (segment (start 193.54 106.79) (end 193.54 130.325685) (width 0.2) (layer "F.Cu") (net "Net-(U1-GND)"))
 (segment (start 144.074899 104.535) (end 144.955 105.415101) (width 0.2) (layer "F.Cu") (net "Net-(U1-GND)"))
 (segment (start 187.945 122.445) (end 187.945 107.655) (width 0.2) (layer "F.Cu") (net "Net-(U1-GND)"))
 (segment (start 186.545 102.815101) (end 187.365101 101.995) (width 0.2) (layer "F.Cu") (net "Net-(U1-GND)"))
 (segment (start 157.96 130.56) (end 149.845 122.445) (width 0.2) (layer "F.Cu") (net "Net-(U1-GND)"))
 (segment (start 187.945 107.655) (end 186.545 106.255) (width 0.2) (layer "F.Cu") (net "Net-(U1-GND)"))
 (segment (start 193.305685 130.56) (end 157.96 130.56) (width 0.2) (layer "F.Cu") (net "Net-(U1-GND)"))
 (segment (start 148.888654 80.94403) (end 129.395 100.437684) (width 0.2) (layer "F.Cu") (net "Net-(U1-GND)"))
 (segment (start 141.915101 105.535) (end 142.915101 104.535) (width 0.2) (layer "F.Cu") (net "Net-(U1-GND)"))
 (segment (start 129.395 105.22) (end 129.71 105.535) (width 0.2) (layer "F.Cu") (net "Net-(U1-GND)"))
 (segment (start 187.365101 101.995) (end 188.745 101.995) (width 0.2) (layer "F.Cu") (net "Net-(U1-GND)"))
 (segment (start 144.955 105.415101) (end 144.955 117.555) (width 0.2) (layer "F.Cu") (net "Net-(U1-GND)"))
 (segment (start 129.395 100.437684) (end 129.395 105.22) (width 0.2) (layer "F.Cu") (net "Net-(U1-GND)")))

